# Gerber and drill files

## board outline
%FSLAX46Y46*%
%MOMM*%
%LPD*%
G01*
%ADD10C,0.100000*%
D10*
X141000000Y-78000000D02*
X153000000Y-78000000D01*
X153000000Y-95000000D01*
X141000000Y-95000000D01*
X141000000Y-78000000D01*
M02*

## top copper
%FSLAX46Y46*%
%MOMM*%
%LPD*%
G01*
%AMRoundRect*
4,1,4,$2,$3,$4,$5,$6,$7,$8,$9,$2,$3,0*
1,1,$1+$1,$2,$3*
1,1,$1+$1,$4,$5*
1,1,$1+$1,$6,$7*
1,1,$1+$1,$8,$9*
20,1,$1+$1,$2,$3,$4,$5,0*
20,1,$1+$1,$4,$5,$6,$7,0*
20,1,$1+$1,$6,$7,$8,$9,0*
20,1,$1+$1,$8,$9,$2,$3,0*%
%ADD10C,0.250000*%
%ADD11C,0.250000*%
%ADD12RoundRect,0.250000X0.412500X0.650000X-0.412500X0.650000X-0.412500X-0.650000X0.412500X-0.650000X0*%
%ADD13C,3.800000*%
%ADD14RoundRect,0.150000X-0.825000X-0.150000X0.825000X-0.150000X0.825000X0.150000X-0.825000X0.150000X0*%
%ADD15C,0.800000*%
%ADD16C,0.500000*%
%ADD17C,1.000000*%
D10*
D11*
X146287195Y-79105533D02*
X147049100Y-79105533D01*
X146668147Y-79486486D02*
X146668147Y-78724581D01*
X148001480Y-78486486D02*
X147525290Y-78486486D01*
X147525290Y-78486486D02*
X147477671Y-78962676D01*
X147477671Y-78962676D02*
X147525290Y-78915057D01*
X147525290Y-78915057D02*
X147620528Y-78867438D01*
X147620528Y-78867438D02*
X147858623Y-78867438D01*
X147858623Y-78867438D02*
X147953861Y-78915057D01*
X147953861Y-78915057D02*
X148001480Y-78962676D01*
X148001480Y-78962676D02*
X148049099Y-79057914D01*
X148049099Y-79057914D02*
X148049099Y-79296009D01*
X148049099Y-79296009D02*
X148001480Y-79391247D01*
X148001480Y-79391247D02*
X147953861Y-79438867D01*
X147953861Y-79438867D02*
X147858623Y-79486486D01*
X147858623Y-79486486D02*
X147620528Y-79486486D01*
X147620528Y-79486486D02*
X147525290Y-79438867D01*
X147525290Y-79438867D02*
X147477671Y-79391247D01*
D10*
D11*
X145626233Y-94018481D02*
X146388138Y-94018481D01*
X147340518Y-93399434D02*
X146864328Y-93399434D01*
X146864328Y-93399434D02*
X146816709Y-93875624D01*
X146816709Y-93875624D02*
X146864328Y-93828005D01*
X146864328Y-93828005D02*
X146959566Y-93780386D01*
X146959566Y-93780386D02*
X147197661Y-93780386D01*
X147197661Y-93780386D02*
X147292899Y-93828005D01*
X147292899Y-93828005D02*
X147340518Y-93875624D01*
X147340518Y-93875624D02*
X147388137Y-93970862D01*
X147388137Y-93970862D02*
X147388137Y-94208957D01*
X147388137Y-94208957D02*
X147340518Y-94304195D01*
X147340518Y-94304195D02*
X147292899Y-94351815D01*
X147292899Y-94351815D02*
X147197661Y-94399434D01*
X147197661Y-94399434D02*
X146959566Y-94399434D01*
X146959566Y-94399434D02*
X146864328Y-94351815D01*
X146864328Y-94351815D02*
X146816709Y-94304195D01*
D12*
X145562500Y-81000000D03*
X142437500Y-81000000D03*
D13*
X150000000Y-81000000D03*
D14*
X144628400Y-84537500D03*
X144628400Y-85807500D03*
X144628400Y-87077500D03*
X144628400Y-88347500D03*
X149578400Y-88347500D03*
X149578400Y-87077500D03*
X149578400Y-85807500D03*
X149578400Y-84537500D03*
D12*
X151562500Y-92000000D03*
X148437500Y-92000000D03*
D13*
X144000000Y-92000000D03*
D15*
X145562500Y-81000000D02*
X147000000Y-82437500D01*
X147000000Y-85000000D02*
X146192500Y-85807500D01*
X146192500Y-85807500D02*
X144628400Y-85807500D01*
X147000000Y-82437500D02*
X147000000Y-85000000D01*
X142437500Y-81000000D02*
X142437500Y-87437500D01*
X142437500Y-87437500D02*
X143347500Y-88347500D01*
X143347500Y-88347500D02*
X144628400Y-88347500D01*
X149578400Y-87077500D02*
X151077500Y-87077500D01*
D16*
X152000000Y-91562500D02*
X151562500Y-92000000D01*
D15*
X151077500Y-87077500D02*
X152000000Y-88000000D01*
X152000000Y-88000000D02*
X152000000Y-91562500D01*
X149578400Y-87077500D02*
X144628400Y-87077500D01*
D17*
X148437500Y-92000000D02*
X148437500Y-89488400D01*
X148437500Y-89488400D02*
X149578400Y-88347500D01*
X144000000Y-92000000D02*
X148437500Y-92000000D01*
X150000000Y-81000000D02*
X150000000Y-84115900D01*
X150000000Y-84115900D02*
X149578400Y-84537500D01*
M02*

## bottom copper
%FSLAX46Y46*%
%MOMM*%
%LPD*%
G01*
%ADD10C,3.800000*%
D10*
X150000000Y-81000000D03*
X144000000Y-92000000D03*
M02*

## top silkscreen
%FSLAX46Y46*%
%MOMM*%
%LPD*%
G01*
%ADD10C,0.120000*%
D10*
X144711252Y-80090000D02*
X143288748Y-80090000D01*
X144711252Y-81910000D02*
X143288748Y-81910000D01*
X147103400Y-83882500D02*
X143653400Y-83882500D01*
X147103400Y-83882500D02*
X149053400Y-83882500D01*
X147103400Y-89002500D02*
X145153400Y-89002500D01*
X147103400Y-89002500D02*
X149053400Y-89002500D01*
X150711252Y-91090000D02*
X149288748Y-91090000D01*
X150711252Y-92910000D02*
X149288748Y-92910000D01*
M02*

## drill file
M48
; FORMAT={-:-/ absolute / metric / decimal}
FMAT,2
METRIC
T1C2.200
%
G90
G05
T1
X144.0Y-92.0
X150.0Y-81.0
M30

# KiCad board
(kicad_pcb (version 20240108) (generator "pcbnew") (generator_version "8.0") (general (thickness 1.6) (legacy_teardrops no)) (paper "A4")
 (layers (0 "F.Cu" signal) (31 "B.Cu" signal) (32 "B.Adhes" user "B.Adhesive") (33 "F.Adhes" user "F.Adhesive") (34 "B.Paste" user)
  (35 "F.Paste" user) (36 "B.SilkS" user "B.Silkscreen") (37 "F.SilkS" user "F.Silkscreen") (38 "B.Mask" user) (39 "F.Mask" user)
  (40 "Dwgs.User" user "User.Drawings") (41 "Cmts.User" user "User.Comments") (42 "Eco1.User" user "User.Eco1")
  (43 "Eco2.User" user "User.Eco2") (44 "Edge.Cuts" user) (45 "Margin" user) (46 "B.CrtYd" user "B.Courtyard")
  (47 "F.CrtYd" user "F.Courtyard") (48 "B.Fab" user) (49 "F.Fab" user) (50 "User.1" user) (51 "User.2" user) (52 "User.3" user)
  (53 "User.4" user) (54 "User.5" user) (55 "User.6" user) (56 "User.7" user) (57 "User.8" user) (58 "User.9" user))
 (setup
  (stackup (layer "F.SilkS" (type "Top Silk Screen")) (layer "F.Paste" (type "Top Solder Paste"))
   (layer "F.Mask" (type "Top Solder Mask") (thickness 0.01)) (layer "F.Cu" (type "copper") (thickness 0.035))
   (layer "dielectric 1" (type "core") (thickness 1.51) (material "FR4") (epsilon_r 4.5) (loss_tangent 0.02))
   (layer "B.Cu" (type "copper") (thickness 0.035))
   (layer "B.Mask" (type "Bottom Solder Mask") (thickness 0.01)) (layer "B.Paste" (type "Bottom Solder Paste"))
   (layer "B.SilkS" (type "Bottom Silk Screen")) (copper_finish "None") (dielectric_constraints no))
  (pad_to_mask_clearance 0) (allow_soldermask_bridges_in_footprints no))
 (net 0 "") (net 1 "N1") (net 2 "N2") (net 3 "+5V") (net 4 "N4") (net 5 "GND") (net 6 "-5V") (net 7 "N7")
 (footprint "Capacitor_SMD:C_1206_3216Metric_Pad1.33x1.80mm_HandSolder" (layer "F.Cu") (at 144 81 180)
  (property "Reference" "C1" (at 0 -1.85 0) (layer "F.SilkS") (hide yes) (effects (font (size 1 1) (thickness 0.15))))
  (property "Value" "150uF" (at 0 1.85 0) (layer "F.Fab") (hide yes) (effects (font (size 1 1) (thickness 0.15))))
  (fp_line (start -0.711252 0.91) (end 0.711252 0.91) (stroke (width 0.12) (type solid)) (layer "F.SilkS"))
  (fp_line (start -0.711252 -0.91) (end 0.711252 -0.91) (stroke (width 0.12) (type solid)) (layer "F.SilkS"))
  (pad "1" smd roundrect (at -1.5625 0 180) (size 1.325 1.8) (layers "F.Cu" "F.Paste" "F.Mask") (roundrect_rratio 0.1886792453) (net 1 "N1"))
  (pad "2" smd roundrect (at 1.5625 0 180) (size 1.325 1.8) (layers "F.Cu" "F.Paste" "F.Mask") (roundrect_rratio 0.1886792453) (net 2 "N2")))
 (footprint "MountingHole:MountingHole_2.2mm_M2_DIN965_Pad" (layer "F.Cu") (at 150 81)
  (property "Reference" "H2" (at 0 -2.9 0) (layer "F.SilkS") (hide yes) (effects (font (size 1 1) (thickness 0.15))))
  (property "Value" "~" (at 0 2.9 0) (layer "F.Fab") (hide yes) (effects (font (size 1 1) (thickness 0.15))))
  (pad "1" thru_hole circle (at 0 0) (size 3.8 3.8) (drill 2.2) (layers "*.Cu" "*.Mask") (remove_unused_layers no) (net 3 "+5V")))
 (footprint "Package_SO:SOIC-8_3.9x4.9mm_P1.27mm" (layer "F.Cu") (at 147.1034 86.4425)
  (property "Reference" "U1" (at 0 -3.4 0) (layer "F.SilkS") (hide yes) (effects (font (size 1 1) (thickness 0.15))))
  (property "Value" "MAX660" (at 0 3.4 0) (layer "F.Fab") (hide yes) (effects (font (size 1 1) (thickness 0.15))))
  (fp_line (start 0 -2.56) (end -3.45 -2.56) (stroke (width 0.12) (type solid)) (layer "F.SilkS"))
  (fp_line (start 0 -2.56) (end 1.95 -2.56) (stroke (width 0.12) (type solid)) (layer "F.SilkS"))
  (fp_line (start 0 2.56) (end -1.95 2.56) (stroke (width 0.12) (type solid)) (layer "F.SilkS"))
  (fp_line (start 0 2.56) (end 1.95 2.56) (stroke (width 0.12) (type solid)) (layer "F.SilkS"))
  (pad "1" smd roundrect (at -2.475 -1.905) (size 1.95 0.6) (layers "F.Cu" "F.Paste" "F.Mask") (roundrect_rratio 0.25) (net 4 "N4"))
  (pad "2" smd roundrect (at -2.475 -0.635) (size 1.95 0.6) (layers "F.Cu" "F.Paste" "F.Mask") (roundrect_rratio 0.25) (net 1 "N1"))
  (pad "3" smd roundrect (at -2.475 0.635) (size 1.95 0.6) (layers "F.Cu" "F.Paste" "F.Mask") (roundrect_rratio 0.25) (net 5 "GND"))
  (pad "4" smd roundrect (at -2.475 1.905) (size 1.95 0.6) (layers "F.Cu" "F.Paste" "F.Mask") (roundrect_rratio 0.25) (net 2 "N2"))
  (pad "5" smd roundrect (at 2.475 1.905) (size 1.95 0.6) (layers "F.Cu" "F.Paste" "F.Mask") (roundrect_rratio 0.25) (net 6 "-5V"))
  (pad "6" smd roundrect (at 2.475 0.635) (size 1.95 0.6) (layers "F.Cu" "F.Paste" "F.Mask") (roundrect_rratio 0.25) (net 5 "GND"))
  (pad "7" smd roundrect (at 2.475 -0.635) (size 1.95 0.6) (layers "F.Cu" "F.Paste" "F.Mask") (roundrect_rratio 0.25) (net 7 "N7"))
  (pad "8" smd roundrect (at 2.475 -1.905) (size 1.95 0.6) (layers "F.Cu" "F.Paste" "F.Mask") (roundrect_rratio 0.25) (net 3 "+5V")))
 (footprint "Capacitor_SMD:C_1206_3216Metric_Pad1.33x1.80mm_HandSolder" (layer "F.Cu") (at 150 92 180)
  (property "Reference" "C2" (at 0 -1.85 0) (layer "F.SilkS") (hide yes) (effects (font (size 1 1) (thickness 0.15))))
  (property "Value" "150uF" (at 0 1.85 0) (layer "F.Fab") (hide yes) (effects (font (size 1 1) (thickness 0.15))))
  (fp_line (start -0.711252 0.91) (end 0.711252 0.91) (stroke (width 0.12) (type solid)) (layer "F.SilkS"))
  (fp_line (start -0.711252 -0.91) (end 0.711252 -0.91) (stroke (width 0.12) (type solid)) (layer "F.SilkS"))
  (pad "1" smd roundrect (at -1.5625 0 180) (size 1.325 1.8) (layers "F.Cu" "F.Paste" "F.Mask") (roundrect_rratio 0.1886792453)
   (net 5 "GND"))
  (pad "2" smd roundrect (at 1.5625 0 180) (size 1.325 1.8) (layers "F.Cu" "F.Paste" "F.Mask") (roundrect_rratio 0.1886792453) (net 6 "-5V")))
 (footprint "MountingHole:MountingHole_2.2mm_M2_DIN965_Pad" (layer "F.Cu") (at 144 92)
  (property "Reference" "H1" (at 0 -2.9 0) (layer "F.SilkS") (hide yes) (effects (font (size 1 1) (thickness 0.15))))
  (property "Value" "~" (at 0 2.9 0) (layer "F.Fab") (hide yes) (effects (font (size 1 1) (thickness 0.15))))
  (pad "1" thru_hole circle (at 0 0) (size 3.8 3.8) (drill 2.2) (layers "*.Cu" "*.Mask") (remove_unused_layers no) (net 6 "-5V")))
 (gr_rect (start 141 78) (end 153 95) (stroke (width 0.1) (type default)) (fill none) (layer "Edge.Cuts"))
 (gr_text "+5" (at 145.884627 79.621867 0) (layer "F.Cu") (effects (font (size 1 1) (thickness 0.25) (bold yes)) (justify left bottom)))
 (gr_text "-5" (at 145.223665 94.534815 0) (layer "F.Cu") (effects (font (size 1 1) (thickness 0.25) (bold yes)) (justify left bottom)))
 (segment (start 145.5625 81) (end 147 82.4375) (width 0.8) (layer "F.Cu") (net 1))
 (segment (start 147 85) (end 146.1925 85.8075) (width 0.8) (layer "F.Cu") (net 1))
 (segment (start 146.1925 85.8075) (end 144.6284 85.8075) (width 0.8) (layer "F.Cu") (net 1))
 (segment (start 147 82.4375) (end 147 85) (width 0.8) (layer "F.Cu") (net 1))
 (segment (start 142.4375 81) (end 142.4375 87.4375) (width 0.8) (layer "F.Cu") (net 2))
 (segment (start 142.4375 87.4375) (end 143.3475 88.3475) (width 0.8) (layer "F.Cu") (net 2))
 (segment (start 143.3475 88.3475) (end 144.6284 88.3475) (width 0.8) (layer "F.Cu") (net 2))
 (segment (start 149.5784 87.0775) (end 151.0775 87.0775) (width 0.8) (layer "F.Cu") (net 5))
 (segment (start 152 91.5625) (end 151.5625 92) (width 0.5) (layer "F.Cu") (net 5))
 (segment (start 151.0775 87.0775) (end 152 88) (width 0.8) (layer "F.Cu") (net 5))
 (segment (start 152 88) (end 152 91.5625) (width 0.8) (layer "F.Cu") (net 5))
 (segment (start 149.5784 87.0775) (end 144.6284 87.0775) (width 0.8) (layer "F.Cu") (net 5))
 (segment (start 148.4375 92) (end 148.4375 89.4884) (width 1) (layer "F.Cu") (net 6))
 (segment (start 148.4375 89.4884) (end 149.5784 88.3475) (width 1) (layer "F.Cu") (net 6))
 (segment (start 144 92) (end 148.4375 92) (width 1) (layer "F.Cu") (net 6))
 (segment (start 150 81) (end 150 84.1159) (width 1) (layer "F.Cu") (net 3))
 (segment (start 150 84.1159) (end 149.5784 84.5375) (width 1) (layer "F.Cu") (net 3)))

